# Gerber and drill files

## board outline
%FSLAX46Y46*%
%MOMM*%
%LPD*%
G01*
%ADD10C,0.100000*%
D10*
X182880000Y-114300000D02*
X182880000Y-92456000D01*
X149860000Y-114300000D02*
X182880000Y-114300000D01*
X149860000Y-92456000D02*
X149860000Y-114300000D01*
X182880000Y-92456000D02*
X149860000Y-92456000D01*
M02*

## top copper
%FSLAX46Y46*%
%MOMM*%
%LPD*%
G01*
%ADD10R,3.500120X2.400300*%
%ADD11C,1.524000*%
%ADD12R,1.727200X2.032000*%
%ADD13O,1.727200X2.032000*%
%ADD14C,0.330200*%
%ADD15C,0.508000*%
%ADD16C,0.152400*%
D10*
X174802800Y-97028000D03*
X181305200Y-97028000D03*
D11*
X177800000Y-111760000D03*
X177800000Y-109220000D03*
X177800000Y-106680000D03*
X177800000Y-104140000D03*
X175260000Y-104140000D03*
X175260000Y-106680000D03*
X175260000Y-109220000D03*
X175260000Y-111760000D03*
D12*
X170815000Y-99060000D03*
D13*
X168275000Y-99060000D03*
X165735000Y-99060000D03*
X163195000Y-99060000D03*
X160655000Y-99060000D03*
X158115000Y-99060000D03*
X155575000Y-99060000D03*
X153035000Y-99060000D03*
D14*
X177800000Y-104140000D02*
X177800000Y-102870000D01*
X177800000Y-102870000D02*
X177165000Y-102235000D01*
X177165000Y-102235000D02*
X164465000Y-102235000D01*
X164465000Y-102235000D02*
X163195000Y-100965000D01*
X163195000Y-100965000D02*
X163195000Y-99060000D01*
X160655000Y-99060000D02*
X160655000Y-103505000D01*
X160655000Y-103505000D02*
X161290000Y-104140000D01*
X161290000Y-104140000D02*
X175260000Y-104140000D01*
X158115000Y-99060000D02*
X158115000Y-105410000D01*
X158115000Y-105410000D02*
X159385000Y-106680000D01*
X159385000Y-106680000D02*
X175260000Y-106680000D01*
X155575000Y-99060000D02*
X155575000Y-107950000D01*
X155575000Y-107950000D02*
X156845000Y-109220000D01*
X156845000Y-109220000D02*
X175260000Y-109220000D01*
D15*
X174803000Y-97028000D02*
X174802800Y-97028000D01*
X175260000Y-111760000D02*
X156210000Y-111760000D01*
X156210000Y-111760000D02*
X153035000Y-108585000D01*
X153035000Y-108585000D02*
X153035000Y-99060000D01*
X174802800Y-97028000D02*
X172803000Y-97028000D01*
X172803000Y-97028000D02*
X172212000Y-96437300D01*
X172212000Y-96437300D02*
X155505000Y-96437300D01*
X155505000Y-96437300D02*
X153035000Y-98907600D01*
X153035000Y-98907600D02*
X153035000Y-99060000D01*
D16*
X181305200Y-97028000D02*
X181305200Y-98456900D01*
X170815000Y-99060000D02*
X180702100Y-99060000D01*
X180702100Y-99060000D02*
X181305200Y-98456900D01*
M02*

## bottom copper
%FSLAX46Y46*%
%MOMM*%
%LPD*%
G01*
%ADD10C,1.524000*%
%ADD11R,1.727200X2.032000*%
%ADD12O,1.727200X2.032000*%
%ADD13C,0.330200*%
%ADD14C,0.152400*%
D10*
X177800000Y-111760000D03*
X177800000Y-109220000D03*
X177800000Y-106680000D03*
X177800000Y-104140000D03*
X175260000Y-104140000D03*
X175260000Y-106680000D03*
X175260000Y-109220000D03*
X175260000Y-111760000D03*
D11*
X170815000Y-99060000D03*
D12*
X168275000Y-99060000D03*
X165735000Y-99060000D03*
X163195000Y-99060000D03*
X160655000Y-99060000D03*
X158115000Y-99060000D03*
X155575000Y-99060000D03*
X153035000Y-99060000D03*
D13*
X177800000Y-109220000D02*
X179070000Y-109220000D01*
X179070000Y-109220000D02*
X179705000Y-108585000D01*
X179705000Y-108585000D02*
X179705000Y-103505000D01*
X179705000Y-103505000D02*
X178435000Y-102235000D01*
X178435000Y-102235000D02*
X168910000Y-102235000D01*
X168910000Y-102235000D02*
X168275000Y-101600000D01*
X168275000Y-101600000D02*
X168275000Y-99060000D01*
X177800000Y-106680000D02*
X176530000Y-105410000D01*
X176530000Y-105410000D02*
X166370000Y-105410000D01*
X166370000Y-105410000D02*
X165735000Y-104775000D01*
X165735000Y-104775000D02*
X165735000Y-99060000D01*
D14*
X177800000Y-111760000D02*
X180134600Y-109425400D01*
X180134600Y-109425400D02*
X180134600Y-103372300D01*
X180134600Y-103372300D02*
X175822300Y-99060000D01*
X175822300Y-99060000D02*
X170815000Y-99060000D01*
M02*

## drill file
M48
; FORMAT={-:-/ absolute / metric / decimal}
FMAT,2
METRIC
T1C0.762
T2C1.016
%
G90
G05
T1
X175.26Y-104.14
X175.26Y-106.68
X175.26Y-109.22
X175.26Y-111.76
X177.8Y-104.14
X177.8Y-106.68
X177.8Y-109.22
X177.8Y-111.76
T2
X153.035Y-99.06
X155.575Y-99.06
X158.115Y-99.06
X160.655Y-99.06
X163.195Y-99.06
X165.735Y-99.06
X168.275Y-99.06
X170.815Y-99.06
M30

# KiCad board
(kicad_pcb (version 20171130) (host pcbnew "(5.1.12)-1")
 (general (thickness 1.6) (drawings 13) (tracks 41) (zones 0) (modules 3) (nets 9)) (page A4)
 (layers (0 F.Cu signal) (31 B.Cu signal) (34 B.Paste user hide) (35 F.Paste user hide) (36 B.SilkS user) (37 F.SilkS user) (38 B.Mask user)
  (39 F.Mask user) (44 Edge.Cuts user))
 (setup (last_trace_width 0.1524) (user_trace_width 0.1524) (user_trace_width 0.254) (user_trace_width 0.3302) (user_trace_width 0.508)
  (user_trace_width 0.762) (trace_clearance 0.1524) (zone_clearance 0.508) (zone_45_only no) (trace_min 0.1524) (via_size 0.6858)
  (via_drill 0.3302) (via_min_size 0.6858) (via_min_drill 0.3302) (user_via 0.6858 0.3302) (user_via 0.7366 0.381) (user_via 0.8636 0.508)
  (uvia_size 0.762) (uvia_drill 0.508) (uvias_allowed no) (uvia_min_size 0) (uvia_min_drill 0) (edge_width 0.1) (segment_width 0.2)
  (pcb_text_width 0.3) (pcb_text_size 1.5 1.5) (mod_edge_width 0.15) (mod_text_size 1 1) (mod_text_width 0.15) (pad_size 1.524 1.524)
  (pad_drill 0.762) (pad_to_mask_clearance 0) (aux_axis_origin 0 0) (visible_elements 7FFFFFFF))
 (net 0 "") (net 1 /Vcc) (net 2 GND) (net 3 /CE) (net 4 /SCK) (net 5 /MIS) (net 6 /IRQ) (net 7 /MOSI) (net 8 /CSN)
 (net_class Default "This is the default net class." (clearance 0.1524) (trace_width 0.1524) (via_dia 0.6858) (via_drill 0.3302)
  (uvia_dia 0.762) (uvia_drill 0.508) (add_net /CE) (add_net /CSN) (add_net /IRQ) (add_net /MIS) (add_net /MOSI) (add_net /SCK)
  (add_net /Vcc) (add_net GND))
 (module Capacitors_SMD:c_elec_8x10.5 (layer F.Cu) (at 178.054 97.028 180)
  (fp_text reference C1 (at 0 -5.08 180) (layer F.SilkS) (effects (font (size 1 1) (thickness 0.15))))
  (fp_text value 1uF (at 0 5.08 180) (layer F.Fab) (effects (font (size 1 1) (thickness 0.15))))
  (pad 1 smd rect (at 3.2512 0 180) (size 3.50012 2.4003) (layers F.Cu F.Paste F.Mask) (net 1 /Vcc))
  (pad 2 smd rect (at -3.2512 0 180) (size 3.50012 2.4003) (layers F.Cu F.Paste F.Mask) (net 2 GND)))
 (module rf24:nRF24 (layer F.Cu) (at 170.18 109.22)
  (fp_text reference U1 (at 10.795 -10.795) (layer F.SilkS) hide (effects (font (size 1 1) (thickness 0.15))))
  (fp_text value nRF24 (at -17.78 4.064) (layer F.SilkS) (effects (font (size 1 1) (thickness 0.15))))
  (pad 0 thru_hole circle (at 7.62 2.54) (size 1.524 1.524) (drill 0.762) (layers *.Cu *.Mask F.SilkS) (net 2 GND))
  (pad 1 thru_hole circle (at 7.62 0) (size 1.524 1.524) (drill 0.762) (layers *.Cu *.Mask F.SilkS) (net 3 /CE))
  (pad 2 thru_hole circle (at 7.62 -2.54) (size 1.524 1.524) (drill 0.762) (layers *.Cu *.Mask F.SilkS) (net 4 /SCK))
  (pad 3 thru_hole circle (at 7.62 -5.08) (size 1.524 1.524) (drill 0.762) (layers *.Cu *.Mask F.SilkS) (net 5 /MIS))
  (pad 4 thru_hole circle (at 5.08 -5.08) (size 1.524 1.524) (drill 0.762) (layers *.Cu *.Mask F.SilkS) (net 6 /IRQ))
  (pad 5 thru_hole circle (at 5.08 -2.54) (size 1.524 1.524) (drill 0.762) (layers *.Cu *.Mask F.SilkS) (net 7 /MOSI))
  (pad 6 thru_hole circle (at 5.08 0) (size 1.524 1.524) (drill 0.762) (layers *.Cu *.Mask F.SilkS) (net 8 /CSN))
  (pad 7 thru_hole circle (at 5.08 2.54) (size 1.524 1.524) (drill 0.762) (layers *.Cu *.Mask F.SilkS) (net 1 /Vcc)))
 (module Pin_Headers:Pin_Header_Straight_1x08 (layer F.Cu) (at 170.815 99.06 270)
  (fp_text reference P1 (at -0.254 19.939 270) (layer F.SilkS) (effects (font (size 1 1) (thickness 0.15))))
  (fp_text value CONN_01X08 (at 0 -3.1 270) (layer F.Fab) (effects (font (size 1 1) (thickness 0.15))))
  (pad 1 thru_hole rect (at 0 0 270) (size 2.032 1.7272) (drill 1.016) (layers *.Cu *.Mask F.SilkS) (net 2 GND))
  (pad 2 thru_hole oval (at 0 2.54 270) (size 2.032 1.7272) (drill 1.016) (layers *.Cu *.Mask F.SilkS) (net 3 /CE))
  (pad 3 thru_hole oval (at 0 5.08 270) (size 2.032 1.7272) (drill 1.016) (layers *.Cu *.Mask F.SilkS) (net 4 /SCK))
  (pad 4 thru_hole oval (at 0 7.62 270) (size 2.032 1.7272) (drill 1.016) (layers *.Cu *.Mask F.SilkS) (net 5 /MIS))
  (pad 5 thru_hole oval (at 0 10.16 270) (size 2.032 1.7272) (drill 1.016) (layers *.Cu *.Mask F.SilkS) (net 6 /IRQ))
  (pad 6 thru_hole oval (at 0 12.7 270) (size 2.032 1.7272) (drill 1.016) (layers *.Cu *.Mask F.SilkS) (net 7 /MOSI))
  (pad 7 thru_hole oval (at 0 15.24 270) (size 2.032 1.7272) (drill 1.016) (layers *.Cu *.Mask F.SilkS) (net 8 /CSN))
  (pad 8 thru_hole oval (at 0 17.78 270) (size 2.032 1.7272) (drill 1.016) (layers *.Cu *.Mask F.SilkS) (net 1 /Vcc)))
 (gr_line (start 182.88 114.3) (end 182.88 92.456) (angle 90) (layer Edge.Cuts) (width 0.1))
 (gr_line (start 149.86 114.3) (end 182.88 114.3) (angle 90) (layer Edge.Cuts) (width 0.1))
 (gr_line (start 149.86 92.456) (end 149.86 114.3) (angle 90) (layer Edge.Cuts) (width 0.1))
 (gr_line (start 182.88 92.456) (end 149.86 92.456) (angle 90) (layer Edge.Cuts) (width 0.1))
 (segment (start 177.8 109.22) (end 179.07 109.22) (width 0.3302) (layer B.Cu) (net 3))
 (segment (start 179.07 109.22) (end 179.705 108.585) (width 0.3302) (layer B.Cu) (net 3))
 (segment (start 179.705 108.585) (end 179.705 103.505) (width 0.3302) (layer B.Cu) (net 3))
 (segment (start 179.705 103.505) (end 178.435 102.235) (width 0.3302) (layer B.Cu) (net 3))
 (segment (start 178.435 102.235) (end 168.91 102.235) (width 0.3302) (layer B.Cu) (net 3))
 (segment (start 168.91 102.235) (end 168.275 101.6) (width 0.3302) (layer B.Cu) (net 3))
 (segment (start 168.275 101.6) (end 168.275 99.06) (width 0.3302) (layer B.Cu) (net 3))
 (segment (start 177.8 106.68) (end 176.53 105.41) (width 0.3302) (layer B.Cu) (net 4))
 (segment (start 176.53 105.41) (end 166.37 105.41) (width 0.3302) (layer B.Cu) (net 4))
 (segment (start 166.37 105.41) (end 165.735 104.775) (width 0.3302) (layer B.Cu) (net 4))
 (segment (start 165.735 104.775) (end 165.735 99.06) (width 0.3302) (layer B.Cu) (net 4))
 (segment (start 177.8 104.14) (end 177.8 102.87) (width 0.3302) (layer F.Cu) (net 5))
 (segment (start 177.8 102.87) (end 177.165 102.235) (width 0.3302) (layer F.Cu) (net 5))
 (segment (start 177.165 102.235) (end 164.465 102.235) (width 0.3302) (layer F.Cu) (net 5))
 (segment (start 164.465 102.235) (end 163.195 100.965) (width 0.3302) (layer F.Cu) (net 5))
 (segment (start 163.195 100.965) (end 163.195 99.06) (width 0.3302) (layer F.Cu) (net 5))
 (segment (start 160.655 99.06) (end 160.655 103.505) (width 0.3302) (layer F.Cu) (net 6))
 (segment (start 160.655 103.505) (end 161.29 104.14) (width 0.3302) (layer F.Cu) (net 6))
 (segment (start 161.29 104.14) (end 175.26 104.14) (width 0.3302) (layer F.Cu) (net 6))
 (segment (start 158.115 99.06) (end 158.115 105.41) (width 0.3302) (layer F.Cu) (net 7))
 (segment (start 158.115 105.41) (end 159.385 106.68) (width 0.3302) (layer F.Cu) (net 7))
 (segment (start 159.385 106.68) (end 175.26 106.68) (width 0.3302) (layer F.Cu) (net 7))
 (segment (start 155.575 99.06) (end 155.575 107.95) (width 0.3302) (layer F.Cu) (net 8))
 (segment (start 155.575 107.95) (end 156.845 109.22) (width 0.3302) (layer F.Cu) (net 8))
 (segment (start 156.845 109.22) (end 175.26 109.22) (width 0.3302) (layer F.Cu) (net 8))
 (segment (start 174.803 97.028) (end 174.8028 97.028) (width 0.508) (layer F.Cu) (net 1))
 (segment (start 175.26 111.76) (end 156.21 111.76) (width 0.508) (layer F.Cu) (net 1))
 (segment (start 156.21 111.76) (end 153.035 108.585) (width 0.508) (layer F.Cu) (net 1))
 (segment (start 153.035 108.585) (end 153.035 99.06) (width 0.508) (layer F.Cu) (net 1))
 (segment (start 174.8028 97.028) (end 172.803 97.028) (width 0.508) (layer F.Cu) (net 1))
 (segment (start 172.803 97.028) (end 172.212 96.4373) (width 0.508) (layer F.Cu) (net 1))
 (segment (start 172.212 96.4373) (end 155.505 96.4373) (width 0.508) (layer F.Cu) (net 1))
 (segment (start 155.505 96.4373) (end 153.035 98.9076) (width 0.508) (layer F.Cu) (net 1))
 (segment (start 153.035 98.9076) (end 153.035 99.06) (width 0.508) (layer F.Cu) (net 1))
 (segment (start 177.8 111.76) (end 180.1346 109.4254) (width 0.1524) (layer B.Cu) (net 2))
 (segment (start 180.1346 109.4254) (end 180.1346 103.3723) (width 0.1524) (layer B.Cu) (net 2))
 (segment (start 180.1346 103.3723) (end 175.8223 99.06) (width 0.1524) (layer B.Cu) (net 2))
 (segment (start 175.8223 99.06) (end 170.815 99.06) (width 0.1524) (layer B.Cu) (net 2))
 (segment (start 181.3052 97.028) (end 181.3052 98.4569) (width 0.1524) (layer F.Cu) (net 2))
 (segment (start 170.815 99.06) (end 180.7021 99.06) (width 0.1524) (layer F.Cu) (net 2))
 (segment (start 180.7021 99.06) (end 181.3052 98.4569) (width 0.1524) (layer F.Cu) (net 2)))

